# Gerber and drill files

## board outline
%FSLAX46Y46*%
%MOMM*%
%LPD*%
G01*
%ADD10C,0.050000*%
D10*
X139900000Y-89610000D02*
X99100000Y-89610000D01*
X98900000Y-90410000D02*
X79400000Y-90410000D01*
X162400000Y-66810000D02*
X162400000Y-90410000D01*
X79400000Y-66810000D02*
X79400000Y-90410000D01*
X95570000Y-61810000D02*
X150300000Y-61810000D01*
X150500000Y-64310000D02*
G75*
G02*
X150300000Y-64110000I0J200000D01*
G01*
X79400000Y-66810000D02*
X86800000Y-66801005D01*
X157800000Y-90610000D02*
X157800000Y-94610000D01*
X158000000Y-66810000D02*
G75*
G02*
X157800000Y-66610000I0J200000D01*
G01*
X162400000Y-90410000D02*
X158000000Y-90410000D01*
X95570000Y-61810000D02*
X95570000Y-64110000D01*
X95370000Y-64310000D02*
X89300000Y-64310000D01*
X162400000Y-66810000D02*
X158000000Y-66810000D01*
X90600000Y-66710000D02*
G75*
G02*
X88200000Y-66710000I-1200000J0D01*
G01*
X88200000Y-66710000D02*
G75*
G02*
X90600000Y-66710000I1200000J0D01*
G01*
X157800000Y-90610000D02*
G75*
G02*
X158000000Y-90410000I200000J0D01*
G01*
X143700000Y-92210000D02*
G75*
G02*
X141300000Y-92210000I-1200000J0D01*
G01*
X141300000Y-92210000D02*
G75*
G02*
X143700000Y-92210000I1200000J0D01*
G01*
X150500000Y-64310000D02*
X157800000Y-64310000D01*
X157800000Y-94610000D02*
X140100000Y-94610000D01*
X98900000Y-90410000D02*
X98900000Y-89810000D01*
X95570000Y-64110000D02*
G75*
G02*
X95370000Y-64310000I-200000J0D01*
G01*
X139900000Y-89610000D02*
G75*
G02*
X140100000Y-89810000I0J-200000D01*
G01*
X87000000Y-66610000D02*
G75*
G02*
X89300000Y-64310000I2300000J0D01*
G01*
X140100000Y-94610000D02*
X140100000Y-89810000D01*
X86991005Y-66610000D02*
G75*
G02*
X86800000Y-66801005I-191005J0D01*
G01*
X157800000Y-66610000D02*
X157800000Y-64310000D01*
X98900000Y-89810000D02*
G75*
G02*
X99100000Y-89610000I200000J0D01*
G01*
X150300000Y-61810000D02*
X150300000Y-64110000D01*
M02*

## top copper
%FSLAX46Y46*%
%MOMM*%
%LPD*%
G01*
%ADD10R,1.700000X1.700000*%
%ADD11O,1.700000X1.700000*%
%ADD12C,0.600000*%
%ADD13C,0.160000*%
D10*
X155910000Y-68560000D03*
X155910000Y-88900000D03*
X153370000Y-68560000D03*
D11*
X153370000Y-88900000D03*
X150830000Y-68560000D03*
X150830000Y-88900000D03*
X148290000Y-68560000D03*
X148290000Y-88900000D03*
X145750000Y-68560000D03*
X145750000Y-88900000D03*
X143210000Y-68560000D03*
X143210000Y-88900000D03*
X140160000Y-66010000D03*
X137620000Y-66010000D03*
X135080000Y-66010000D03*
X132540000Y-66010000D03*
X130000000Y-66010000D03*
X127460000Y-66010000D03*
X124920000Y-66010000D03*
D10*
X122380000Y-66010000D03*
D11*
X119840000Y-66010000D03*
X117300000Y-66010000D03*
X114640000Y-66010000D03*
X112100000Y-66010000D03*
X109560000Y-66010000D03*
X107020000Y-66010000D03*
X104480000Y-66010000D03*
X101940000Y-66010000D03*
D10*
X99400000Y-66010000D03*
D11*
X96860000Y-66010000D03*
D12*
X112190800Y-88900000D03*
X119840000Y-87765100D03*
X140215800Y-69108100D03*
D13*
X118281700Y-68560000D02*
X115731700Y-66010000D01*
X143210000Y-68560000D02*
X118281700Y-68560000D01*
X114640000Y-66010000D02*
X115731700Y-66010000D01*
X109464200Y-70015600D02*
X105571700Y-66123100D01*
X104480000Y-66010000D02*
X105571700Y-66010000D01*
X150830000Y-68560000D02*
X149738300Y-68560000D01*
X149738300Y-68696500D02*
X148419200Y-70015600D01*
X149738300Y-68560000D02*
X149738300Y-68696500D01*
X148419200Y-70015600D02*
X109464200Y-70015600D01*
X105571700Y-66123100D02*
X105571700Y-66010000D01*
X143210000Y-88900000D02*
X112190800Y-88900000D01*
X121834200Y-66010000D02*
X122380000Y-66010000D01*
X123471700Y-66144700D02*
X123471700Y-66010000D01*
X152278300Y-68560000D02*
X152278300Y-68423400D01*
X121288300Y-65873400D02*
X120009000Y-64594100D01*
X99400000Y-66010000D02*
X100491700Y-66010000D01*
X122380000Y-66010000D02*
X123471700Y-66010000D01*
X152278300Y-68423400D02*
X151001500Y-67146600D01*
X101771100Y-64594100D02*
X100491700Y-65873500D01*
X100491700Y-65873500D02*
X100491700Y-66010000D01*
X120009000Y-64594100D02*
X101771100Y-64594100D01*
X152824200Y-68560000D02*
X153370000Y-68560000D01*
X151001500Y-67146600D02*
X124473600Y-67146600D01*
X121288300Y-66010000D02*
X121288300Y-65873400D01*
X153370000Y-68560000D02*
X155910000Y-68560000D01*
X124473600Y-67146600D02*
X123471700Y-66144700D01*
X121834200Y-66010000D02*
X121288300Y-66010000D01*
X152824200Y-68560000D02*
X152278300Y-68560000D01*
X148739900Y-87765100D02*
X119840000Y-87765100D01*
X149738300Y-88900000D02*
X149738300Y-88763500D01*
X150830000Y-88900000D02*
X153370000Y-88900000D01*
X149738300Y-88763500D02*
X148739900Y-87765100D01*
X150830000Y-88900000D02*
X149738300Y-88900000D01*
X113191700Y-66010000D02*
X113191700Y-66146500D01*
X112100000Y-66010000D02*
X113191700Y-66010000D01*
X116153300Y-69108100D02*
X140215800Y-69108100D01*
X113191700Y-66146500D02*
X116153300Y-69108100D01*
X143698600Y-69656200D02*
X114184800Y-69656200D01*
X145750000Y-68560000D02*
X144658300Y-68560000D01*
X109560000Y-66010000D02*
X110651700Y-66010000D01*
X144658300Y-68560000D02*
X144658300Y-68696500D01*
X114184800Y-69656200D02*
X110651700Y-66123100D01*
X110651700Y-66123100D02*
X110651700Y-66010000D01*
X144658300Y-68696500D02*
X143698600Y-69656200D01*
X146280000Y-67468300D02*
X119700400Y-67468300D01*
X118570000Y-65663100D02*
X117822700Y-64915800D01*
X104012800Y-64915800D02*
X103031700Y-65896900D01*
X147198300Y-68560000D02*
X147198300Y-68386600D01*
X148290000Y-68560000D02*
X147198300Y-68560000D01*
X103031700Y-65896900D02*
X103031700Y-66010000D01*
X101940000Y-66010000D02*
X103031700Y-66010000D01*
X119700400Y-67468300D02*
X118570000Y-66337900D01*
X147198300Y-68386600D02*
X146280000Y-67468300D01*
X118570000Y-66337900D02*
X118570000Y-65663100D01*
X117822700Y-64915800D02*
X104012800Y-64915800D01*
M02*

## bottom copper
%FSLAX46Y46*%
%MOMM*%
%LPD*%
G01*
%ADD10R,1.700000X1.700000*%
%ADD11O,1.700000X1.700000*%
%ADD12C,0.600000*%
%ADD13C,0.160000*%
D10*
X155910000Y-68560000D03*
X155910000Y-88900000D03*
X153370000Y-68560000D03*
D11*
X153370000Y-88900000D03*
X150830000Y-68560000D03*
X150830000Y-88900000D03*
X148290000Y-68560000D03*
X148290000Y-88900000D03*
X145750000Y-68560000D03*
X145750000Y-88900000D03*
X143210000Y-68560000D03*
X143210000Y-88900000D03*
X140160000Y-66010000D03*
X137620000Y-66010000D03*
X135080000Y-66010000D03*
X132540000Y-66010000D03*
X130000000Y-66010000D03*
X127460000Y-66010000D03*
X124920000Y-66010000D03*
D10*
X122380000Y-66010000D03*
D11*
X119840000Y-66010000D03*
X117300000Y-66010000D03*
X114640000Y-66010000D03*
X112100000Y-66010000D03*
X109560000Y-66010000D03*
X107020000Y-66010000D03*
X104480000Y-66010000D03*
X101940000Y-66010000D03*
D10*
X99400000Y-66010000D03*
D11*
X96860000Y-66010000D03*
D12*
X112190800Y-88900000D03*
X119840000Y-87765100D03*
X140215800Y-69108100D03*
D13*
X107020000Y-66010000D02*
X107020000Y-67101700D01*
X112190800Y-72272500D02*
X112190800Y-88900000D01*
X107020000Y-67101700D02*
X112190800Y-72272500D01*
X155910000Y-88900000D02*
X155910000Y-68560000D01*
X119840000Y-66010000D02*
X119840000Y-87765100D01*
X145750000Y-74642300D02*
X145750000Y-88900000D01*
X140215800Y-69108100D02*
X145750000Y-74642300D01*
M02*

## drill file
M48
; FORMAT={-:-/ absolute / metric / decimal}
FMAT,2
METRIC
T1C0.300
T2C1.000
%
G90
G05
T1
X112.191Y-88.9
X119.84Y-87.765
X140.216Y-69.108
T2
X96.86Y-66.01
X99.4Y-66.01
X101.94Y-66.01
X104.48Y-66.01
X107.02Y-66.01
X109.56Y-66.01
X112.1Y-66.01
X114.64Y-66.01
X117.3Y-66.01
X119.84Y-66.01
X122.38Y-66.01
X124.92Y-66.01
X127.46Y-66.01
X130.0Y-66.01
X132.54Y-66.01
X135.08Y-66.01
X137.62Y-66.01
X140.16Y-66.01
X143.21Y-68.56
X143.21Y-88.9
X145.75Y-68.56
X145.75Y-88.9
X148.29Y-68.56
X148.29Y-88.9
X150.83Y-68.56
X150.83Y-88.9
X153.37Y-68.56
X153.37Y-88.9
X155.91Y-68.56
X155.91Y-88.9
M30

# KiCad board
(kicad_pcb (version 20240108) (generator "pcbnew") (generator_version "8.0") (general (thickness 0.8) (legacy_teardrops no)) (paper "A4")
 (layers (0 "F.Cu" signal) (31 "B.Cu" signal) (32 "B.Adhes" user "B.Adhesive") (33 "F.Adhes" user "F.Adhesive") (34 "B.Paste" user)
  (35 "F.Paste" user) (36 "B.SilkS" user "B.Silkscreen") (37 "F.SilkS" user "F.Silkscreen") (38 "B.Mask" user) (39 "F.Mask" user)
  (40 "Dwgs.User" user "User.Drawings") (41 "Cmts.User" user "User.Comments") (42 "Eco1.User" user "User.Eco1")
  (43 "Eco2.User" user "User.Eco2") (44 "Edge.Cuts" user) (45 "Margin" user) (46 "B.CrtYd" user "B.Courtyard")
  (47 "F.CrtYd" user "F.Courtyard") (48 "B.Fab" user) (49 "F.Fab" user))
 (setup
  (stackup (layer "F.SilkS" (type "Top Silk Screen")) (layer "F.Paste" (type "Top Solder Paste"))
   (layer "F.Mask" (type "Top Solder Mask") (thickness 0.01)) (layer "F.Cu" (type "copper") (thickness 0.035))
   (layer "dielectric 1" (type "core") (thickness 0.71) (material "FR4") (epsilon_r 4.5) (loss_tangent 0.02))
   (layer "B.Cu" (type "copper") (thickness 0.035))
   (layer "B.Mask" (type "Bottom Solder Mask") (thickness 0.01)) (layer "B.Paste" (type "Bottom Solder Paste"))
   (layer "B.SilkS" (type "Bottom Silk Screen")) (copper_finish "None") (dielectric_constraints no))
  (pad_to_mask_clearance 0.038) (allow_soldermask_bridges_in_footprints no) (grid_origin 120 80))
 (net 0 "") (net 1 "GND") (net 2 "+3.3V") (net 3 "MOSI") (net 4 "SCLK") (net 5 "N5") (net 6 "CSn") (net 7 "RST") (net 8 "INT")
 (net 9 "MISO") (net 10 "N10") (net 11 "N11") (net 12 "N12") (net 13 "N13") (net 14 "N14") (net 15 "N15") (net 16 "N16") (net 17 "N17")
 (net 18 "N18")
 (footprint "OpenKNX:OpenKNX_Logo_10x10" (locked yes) (layer "F.Cu") (at 150.39 91.63)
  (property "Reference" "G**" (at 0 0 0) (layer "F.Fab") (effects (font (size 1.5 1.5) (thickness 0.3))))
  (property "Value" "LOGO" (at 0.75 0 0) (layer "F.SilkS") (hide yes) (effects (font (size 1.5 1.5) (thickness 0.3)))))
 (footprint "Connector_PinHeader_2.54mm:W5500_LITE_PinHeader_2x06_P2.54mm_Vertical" (layer "F.Cu") (at 155.91 86.36 -90)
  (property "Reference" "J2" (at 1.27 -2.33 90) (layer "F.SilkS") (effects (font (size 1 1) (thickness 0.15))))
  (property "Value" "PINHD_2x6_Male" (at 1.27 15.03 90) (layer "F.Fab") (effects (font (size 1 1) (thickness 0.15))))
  (pad "1" thru_hole rect (at -17.8 0 270) (size 1.7 1.7) (drill 1) (layers "*.Cu" "*.Mask") (remove_unused_layers no) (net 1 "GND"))
  (pad "2" thru_hole rect (at 2.54 0 270) (size 1.7 1.7) (drill 1) (layers "*.Cu" "*.Mask") (remove_unused_layers no) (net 1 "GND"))
  (pad "3" thru_hole rect (at -17.8 2.54 270) (size 1.7 1.7) (drill 1) (layers "*.Cu" "*.Mask") (remove_unused_layers no) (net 1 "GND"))
  (pad "4" thru_hole oval (at 2.54 2.54 270) (size 1.7 1.7) (drill 1) (layers "*.Cu" "*.Mask") (remove_unused_layers no) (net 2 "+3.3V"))
  (pad "5" thru_hole oval (at -17.8 5.08 270) (size 1.7 1.7) (drill 1) (layers "*.Cu" "*.Mask") (remove_unused_layers no) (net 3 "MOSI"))
  (pad "6" thru_hole oval (at 2.54 5.08 270) (size 1.7 1.7) (drill 1) (layers "*.Cu" "*.Mask") (remove_unused_layers no) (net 2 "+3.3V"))
  (pad "7" thru_hole oval (at -17.8 7.62 270) (size 1.7 1.7) (drill 1) (layers "*.Cu" "*.Mask") (remove_unused_layers no) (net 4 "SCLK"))
  (pad "8" thru_hole oval (at 2.54 7.62 270) (size 1.7 1.7) (drill 1) (layers "*.Cu" "*.Mask") (remove_unused_layers no) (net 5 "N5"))
  (pad "9" thru_hole oval (at -17.8 10.16 270) (size 1.7 1.7) (drill 1) (layers "*.Cu" "*.Mask") (remove_unused_layers no) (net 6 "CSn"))
  (pad "10" thru_hole oval (at 2.54 10.16 270) (size 1.7 1.7) (drill 1) (layers "*.Cu" "*.Mask") (remove_unused_layers no) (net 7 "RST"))
  (pad "11" thru_hole oval (at -17.8 12.7 270) (size 1.7 1.7) (drill 1) (layers "*.Cu" "*.Mask") (remove_unused_layers no) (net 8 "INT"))
  (pad "12" thru_hole oval (at 2.54 12.7 270) (size 1.7 1.7) (drill 1) (layers "*.Cu" "*.Mask") (remove_unused_layers no) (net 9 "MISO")))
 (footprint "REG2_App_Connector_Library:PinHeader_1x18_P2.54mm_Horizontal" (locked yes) (layer "B.Cu") (at 140.16 66.01 90)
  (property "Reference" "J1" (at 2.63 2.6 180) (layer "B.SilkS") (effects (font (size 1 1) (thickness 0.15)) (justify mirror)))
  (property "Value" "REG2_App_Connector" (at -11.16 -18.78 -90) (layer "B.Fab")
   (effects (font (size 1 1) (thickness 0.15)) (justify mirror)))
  (pad "1" thru_hole oval (at 0 0 90) (size 1.7 1.7) (drill 1) (layers "*.Cu" "*.Mask") (remove_unused_layers no) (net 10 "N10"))
  (pad "2" thru_hole oval (at 0 -2.54 90) (size 1.7 1.7) (drill 1) (layers "*.Cu" "*.Mask") (remove_unused_layers no) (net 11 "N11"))
  (pad "3" thru_hole oval (at 0 -5.08 90) (size 1.7 1.7) (drill 1) (layers "*.Cu" "*.Mask") (remove_unused_layers no) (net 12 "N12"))
  (pad "4" thru_hole oval (at 0 -7.62 90) (size 1.7 1.7) (drill 1) (layers "*.Cu" "*.Mask") (remove_unused_layers no) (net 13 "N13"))
  (pad "5" thru_hole oval (at 0 -10.16 90) (size 1.7 1.7) (drill 1) (layers "*.Cu" "*.Mask") (remove_unused_layers no) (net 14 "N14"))
  (pad "6" thru_hole oval (at 0 -12.7 90) (size 1.7 1.7) (drill 1) (layers "*.Cu" "*.Mask") (remove_unused_layers no) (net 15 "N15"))
  (pad "7" thru_hole oval (at 0 -15.24 90) (size 1.7 1.7) (drill 1) (layers "*.Cu" "*.Mask") (remove_unused_layers no) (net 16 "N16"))
  (pad "8" thru_hole rect (at 0 -17.78 90) (size 1.7 1.7) (drill 1) (layers "*.Cu" "*.Mask") (remove_unused_layers no) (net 1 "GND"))
  (pad "9" thru_hole oval (at 0 -20.32 90) (size 1.7 1.7) (drill 1) (layers "*.Cu" "*.Mask") (remove_unused_layers no) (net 2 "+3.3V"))
  (pad "10" thru_hole oval (at 0 -22.86 90) (size 1.7 1.7) (drill 1) (layers "*.Cu" "*.Mask") (remove_unused_layers no) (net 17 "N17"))
  (pad "11" thru_hole oval (at 0 -25.52 90) (size 1.7 1.7) (drill 1) (layers "*.Cu" "*.Mask") (remove_unused_layers no) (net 8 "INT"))
  (pad "12" thru_hole oval (at 0 -28.06 90) (size 1.7 1.7) (drill 1) (layers "*.Cu" "*.Mask") (remove_unused_layers no) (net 7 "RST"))
  (pad "13" thru_hole oval (at 0 -30.6 90) (size 1.7 1.7) (drill 1) (layers "*.Cu" "*.Mask") (remove_unused_layers no) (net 6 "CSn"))
  (pad "14" thru_hole oval (at 0 -33.14 90) (size 1.7 1.7) (drill 1) (layers "*.Cu" "*.Mask") (remove_unused_layers no) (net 9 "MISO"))
  (pad "15" thru_hole oval (at 0 -35.68 90) (size 1.7 1.7) (drill 1) (layers "*.Cu" "*.Mask") (remove_unused_layers no) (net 3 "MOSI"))
  (pad "16" thru_hole oval (at 0 -38.22 90) (size 1.7 1.7) (drill 1) (layers "*.Cu" "*.Mask") (remove_unused_layers no) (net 4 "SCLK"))
  (pad "17" thru_hole rect (at 0 -40.76 90) (size 1.7 1.7) (drill 1) (layers "*.Cu" "*.Mask") (remove_unused_layers no) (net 1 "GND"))
  (pad "18" thru_hole oval (at 0 -43.3 90) (size 1.7 1.7) (drill 1) (layers "*.Cu" "*.Mask") (remove_unused_layers no) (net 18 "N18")))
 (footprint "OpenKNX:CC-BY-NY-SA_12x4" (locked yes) (layer "B.Cu") (at 101.024889 71.165111 180)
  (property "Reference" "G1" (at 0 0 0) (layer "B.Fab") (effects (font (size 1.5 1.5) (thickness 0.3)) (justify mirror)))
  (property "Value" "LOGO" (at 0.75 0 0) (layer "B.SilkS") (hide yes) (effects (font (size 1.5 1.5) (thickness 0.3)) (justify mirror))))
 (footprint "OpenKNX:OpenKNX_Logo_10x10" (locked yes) (layer "B.Cu") (at 138.16 71.14 180)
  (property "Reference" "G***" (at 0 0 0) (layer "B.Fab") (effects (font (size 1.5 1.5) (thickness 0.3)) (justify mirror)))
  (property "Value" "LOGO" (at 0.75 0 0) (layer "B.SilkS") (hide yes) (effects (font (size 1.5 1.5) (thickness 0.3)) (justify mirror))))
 (gr_line (start 139.9 89.61) (end 99.1 89.61) (stroke (width 0.05) (type solid)) (layer "Edge.Cuts"))
 (gr_line (start 98.9 90.41) (end 79.4 90.41) (stroke (width 0.05) (type solid)) (layer "Edge.Cuts"))
 (gr_line (start 162.4 66.81) (end 162.4 90.41) (stroke (width 0.05) (type solid)) (layer "Edge.Cuts"))
 (gr_line (start 79.4 66.81) (end 79.4 90.41) (stroke (width 0.05) (type solid)) (layer "Edge.Cuts"))
 (gr_line (start 95.57 61.81) (end 150.3 61.81) (stroke (width 0.05) (type solid)) (layer "Edge.Cuts"))
 (gr_arc (start 150.5 64.31) (mid 150.358579 64.251421) (end 150.3 64.11) (stroke (width 0.05) (type solid)) (layer "Edge.Cuts"))
 (gr_line (start 79.4 66.81) (end 86.8 66.801005) (stroke (width 0.05) (type solid)) (layer "Edge.Cuts"))
 (gr_line (start 157.8 90.61) (end 157.8 94.61) (stroke (width 0.05) (type solid)) (layer "Edge.Cuts"))
 (gr_arc (start 158 66.81) (mid 157.858579 66.751421) (end 157.8 66.61) (stroke (width 0.05) (type solid)) (layer "Edge.Cuts"))
 (gr_line (start 162.4 90.41) (end 158 90.41) (stroke (width 0.05) (type solid)) (layer "Edge.Cuts"))
 (gr_line (start 95.57 61.81) (end 95.57 64.11) (stroke (width 0.05) (type solid)) (layer "Edge.Cuts"))
 (gr_line (start 95.37 64.31) (end 89.3 64.31) (stroke (width 0.05) (type solid)) (layer "Edge.Cuts"))
 (gr_line (start 162.4 66.81) (end 158 66.81) (stroke (width 0.05) (type solid)) (layer "Edge.Cuts"))
 (gr_circle (center 89.4 66.71) (end 90.6 66.71) (stroke (width 0.05) (type solid)) (fill none) (layer "Edge.Cuts"))
 (gr_arc (start 157.8 90.61) (mid 157.858579 90.468579) (end 158 90.41) (stroke (width 0.05) (type solid)) (layer "Edge.Cuts"))
 (gr_circle (center 142.5 92.21) (end 142.5 93.41) (stroke (width 0.05) (type solid)) (fill none) (layer "Edge.Cuts"))
 (gr_line (start 150.5 64.31) (end 157.8 64.31) (stroke (width 0.05) (type default)) (layer "Edge.Cuts"))
 (gr_line (start 157.8 94.61) (end 140.1 94.61) (stroke (width 0.05) (type solid)) (layer "Edge.Cuts"))
 (gr_line (start 98.9 90.41) (end 98.9 89.81) (stroke (width 0.05) (type default)) (layer "Edge.Cuts"))
 (gr_arc (start 95.57 64.11) (mid 95.511421 64.251421) (end 95.37 64.31) (stroke (width 0.05) (type default)) (layer "Edge.Cuts"))
 (gr_arc (start 139.9 89.61) (mid 140.041421 89.668579) (end 140.1 89.81) (stroke (width 0.05) (type solid)) (layer "Edge.Cuts"))
 (gr_arc (start 87 66.61) (mid 87.673654 64.983654) (end 89.3 64.31) (stroke (width 0.05) (type default)) (layer "Edge.Cuts"))
 (gr_line (start 140.1 94.61) (end 140.1 89.81) (stroke (width 0.05) (type solid)) (layer "Edge.Cuts"))
 (gr_arc (start 86.991005 66.61) (mid 86.935061 66.745061) (end 86.8 66.801005) (stroke (width 0.05) (type default)) (layer "Edge.Cuts"))
 (gr_line (start 157.8 66.61) (end 157.8 64.31) (stroke (width 0.05) (type solid)) (layer "Edge.Cuts"))
 (gr_arc (start 98.9 89.81) (mid 98.958579 89.668579) (end 99.1 89.61) (stroke (width 0.05) (type solid)) (layer "Edge.Cuts"))
 (gr_line (start 150.3 61.81) (end 150.3 64.11) (stroke (width 0.05) (type solid)) (layer "Edge.Cuts"))
 (segment (start 118.2817 68.56) (end 115.7317 66.01) (width 0.16) (layer "F.Cu") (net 8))
 (segment (start 143.21 68.56) (end 118.2817 68.56) (width 0.16) (layer "F.Cu") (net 8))
 (segment (start 114.64 66.01) (end 115.7317 66.01) (width 0.16) (layer "F.Cu") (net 8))
 (segment (start 109.4642 70.0156) (end 105.5717 66.1231) (width 0.16) (layer "F.Cu") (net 3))
 (segment (start 104.48 66.01) (end 105.5717 66.01) (width 0.16) (layer "F.Cu") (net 3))
 (segment (start 150.83 68.56) (end 149.7383 68.56) (width 0.16) (layer "F.Cu") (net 3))
 (segment (start 149.7383 68.6965) (end 148.4192 70.0156) (width 0.16) (layer "F.Cu") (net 3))
 (segment (start 149.7383 68.56) (end 149.7383 68.6965) (width 0.16) (layer "F.Cu") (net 3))
 (segment (start 148.4192 70.0156) (end 109.4642 70.0156) (width 0.16) (layer "F.Cu") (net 3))
 (segment (start 105.5717 66.1231) (end 105.5717 66.01) (width 0.16) (layer "F.Cu") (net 3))
 (segment (start 143.21 88.9) (end 112.1908 88.9) (width 0.16) (layer "F.Cu") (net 9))
 (via (at 112.1908 88.9) (size 0.6) (drill 0.3) (layers "F.Cu" "B.Cu") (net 9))
 (segment (start 107.02 66.01) (end 107.02 67.1017) (width 0.16) (layer "B.Cu") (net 9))
 (segment (start 112.1908 72.2725) (end 112.1908 88.9) (width 0.16) (layer "B.Cu") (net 9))
 (segment (start 107.02 67.1017) (end 112.1908 72.2725) (width 0.16) (layer "B.Cu") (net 9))
 (segment (start 121.8342 66.01) (end 122.38 66.01) (width 0.16) (layer "F.Cu") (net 1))
 (segment (start 123.4717 66.1447) (end 123.4717 66.01) (width 0.16) (layer "F.Cu") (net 1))
 (segment (start 152.2783 68.56) (end 152.2783 68.4234) (width 0.16) (layer "F.Cu") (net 1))
 (segment (start 121.2883 65.8734) (end 120.009 64.5941) (width 0.16) (layer "F.Cu") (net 1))
 (segment (start 99.4 66.01) (end 100.4917 66.01) (width 0.16) (layer "F.Cu") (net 1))
 (segment (start 122.38 66.01) (end 123.4717 66.01) (width 0.16) (layer "F.Cu") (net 1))
 (segment (start 152.2783 68.4234) (end 151.0015 67.1466) (width 0.16) (layer "F.Cu") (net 1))
 (segment (start 101.7711 64.5941) (end 100.4917 65.8735) (width 0.16) (layer "F.Cu") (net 1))
 (segment (start 100.4917 65.8735) (end 100.4917 66.01) (width 0.16) (layer "F.Cu") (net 1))
 (segment (start 120.009 64.5941) (end 101.7711 64.5941) (width 0.16) (layer "F.Cu") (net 1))
 (segment (start 152.8242 68.56) (end 153.37 68.56) (width 0.16) (layer "F.Cu") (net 1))
 (segment (start 151.0015 67.1466) (end 124.4736 67.1466) (width 0.16) (layer "F.Cu") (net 1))
 (segment (start 121.2883 66.01) (end 121.2883 65.8734) (width 0.16) (layer "F.Cu") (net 1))
 (segment (start 153.37 68.56) (end 155.91 68.56) (width 0.16) (layer "F.Cu") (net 1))
 (segment (start 124.4736 67.1466) (end 123.4717 66.1447) (width 0.16) (layer "F.Cu") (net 1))
 (segment (start 121.8342 66.01) (end 121.2883 66.01) (width 0.16) (layer "F.Cu") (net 1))
 (segment (start 152.8242 68.56) (end 152.2783 68.56) (width 0.16) (layer "F.Cu") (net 1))
 (segment (start 155.91 88.9) (end 155.91 68.56) (width 0.16) (layer "B.Cu") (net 1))
 (segment (start 148.7399 87.7651) (end 119.84 87.7651) (width 0.16) (layer "F.Cu") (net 2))
 (segment (start 149.7383 88.9) (end 149.7383 88.7635) (width 0.16) (layer "F.Cu") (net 2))
 (segment (start 150.83 88.9) (end 153.37 88.9) (width 0.16) (layer "F.Cu") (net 2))
 (segment (start 149.7383 88.7635) (end 148.7399 87.7651) (width 0.16) (layer "F.Cu") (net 2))
 (segment (start 150.83 88.9) (end 149.7383 88.9) (width 0.16) (layer "F.Cu") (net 2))
 (via (at 119.84 87.7651) (size 0.6) (drill 0.3) (layers "F.Cu" "B.Cu") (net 2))
 (segment (start 119.84 66.01) (end 119.84 87.7651) (width 0.16) (layer "B.Cu") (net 2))
 (segment (start 113.1917 66.01) (end 113.1917 66.1465) (width 0.16) (layer "F.Cu") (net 7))
 (segment (start 112.1 66.01) (end 113.1917 66.01) (width 0.16) (layer "F.Cu") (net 7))
 (segment (start 116.1533 69.1081) (end 140.2158 69.1081) (width 0.16) (layer "F.Cu") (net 7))
 (segment (start 113.1917 66.1465) (end 116.1533 69.1081) (width 0.16) (layer "F.Cu") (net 7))
 (via (at 140.2158 69.1081) (size 0.6) (drill 0.3) (layers "F.Cu" "B.Cu") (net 7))
 (segment (start 145.75 74.6423) (end 145.75 88.9) (width 0.16) (layer "B.Cu") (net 7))
 (segment (start 140.2158 69.1081) (end 145.75 74.6423) (width 0.16) (layer "B.Cu") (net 7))
 (segment (start 143.6986 69.6562) (end 114.1848 69.6562) (width 0.16) (layer "F.Cu") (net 6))
 (segment (start 145.75 68.56) (end 144.6583 68.56) (width 0.16) (layer "F.Cu") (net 6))
 (segment (start 109.56 66.01) (end 110.6517 66.01) (width 0.16) (layer "F.Cu") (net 6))
 (segment (start 144.6583 68.56) (end 144.6583 68.6965) (width 0.16) (layer "F.Cu") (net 6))
 (segment (start 114.1848 69.6562) (end 110.6517 66.1231) (width 0.16) (layer "F.Cu") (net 6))
 (segment (start 110.6517 66.1231) (end 110.6517 66.01) (width 0.16) (layer "F.Cu") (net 6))
 (segment (start 144.6583 68.6965) (end 143.6986 69.6562) (width 0.16) (layer "F.Cu") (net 6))
 (segment (start 146.28 67.4683) (end 119.7004 67.4683) (width 0.16) (layer "F.Cu") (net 4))
 (segment (start 118.57 65.6631) (end 117.8227 64.9158) (width 0.16) (layer "F.Cu") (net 4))
 (segment (start 104.0128 64.9158) (end 103.0317 65.8969) (width 0.16) (layer "F.Cu") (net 4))
 (segment (start 147.1983 68.56) (end 147.1983 68.3866) (width 0.16) (layer "F.Cu") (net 4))
 (segment (start 148.29 68.56) (end 147.1983 68.56) (width 0.16) (layer "F.Cu") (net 4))
 (segment (start 103.0317 65.8969) (end 103.0317 66.01) (width 0.16) (layer "F.Cu") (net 4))
 (segment (start 101.94 66.01) (end 103.0317 66.01) (width 0.16) (layer "F.Cu") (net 4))
 (segment (start 119.7004 67.4683) (end 118.57 66.3379) (width 0.16) (layer "F.Cu") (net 4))
 (segment (start 147.1983 68.3866) (end 146.28 67.4683) (width 0.16) (layer "F.Cu") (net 4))
 (segment (start 118.57 66.3379) (end 118.57 65.6631) (width 0.16) (layer "F.Cu") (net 4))
 (segment (start 117.8227 64.9158) (end 104.0128 64.9158) (width 0.16) (layer "F.Cu") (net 4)))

